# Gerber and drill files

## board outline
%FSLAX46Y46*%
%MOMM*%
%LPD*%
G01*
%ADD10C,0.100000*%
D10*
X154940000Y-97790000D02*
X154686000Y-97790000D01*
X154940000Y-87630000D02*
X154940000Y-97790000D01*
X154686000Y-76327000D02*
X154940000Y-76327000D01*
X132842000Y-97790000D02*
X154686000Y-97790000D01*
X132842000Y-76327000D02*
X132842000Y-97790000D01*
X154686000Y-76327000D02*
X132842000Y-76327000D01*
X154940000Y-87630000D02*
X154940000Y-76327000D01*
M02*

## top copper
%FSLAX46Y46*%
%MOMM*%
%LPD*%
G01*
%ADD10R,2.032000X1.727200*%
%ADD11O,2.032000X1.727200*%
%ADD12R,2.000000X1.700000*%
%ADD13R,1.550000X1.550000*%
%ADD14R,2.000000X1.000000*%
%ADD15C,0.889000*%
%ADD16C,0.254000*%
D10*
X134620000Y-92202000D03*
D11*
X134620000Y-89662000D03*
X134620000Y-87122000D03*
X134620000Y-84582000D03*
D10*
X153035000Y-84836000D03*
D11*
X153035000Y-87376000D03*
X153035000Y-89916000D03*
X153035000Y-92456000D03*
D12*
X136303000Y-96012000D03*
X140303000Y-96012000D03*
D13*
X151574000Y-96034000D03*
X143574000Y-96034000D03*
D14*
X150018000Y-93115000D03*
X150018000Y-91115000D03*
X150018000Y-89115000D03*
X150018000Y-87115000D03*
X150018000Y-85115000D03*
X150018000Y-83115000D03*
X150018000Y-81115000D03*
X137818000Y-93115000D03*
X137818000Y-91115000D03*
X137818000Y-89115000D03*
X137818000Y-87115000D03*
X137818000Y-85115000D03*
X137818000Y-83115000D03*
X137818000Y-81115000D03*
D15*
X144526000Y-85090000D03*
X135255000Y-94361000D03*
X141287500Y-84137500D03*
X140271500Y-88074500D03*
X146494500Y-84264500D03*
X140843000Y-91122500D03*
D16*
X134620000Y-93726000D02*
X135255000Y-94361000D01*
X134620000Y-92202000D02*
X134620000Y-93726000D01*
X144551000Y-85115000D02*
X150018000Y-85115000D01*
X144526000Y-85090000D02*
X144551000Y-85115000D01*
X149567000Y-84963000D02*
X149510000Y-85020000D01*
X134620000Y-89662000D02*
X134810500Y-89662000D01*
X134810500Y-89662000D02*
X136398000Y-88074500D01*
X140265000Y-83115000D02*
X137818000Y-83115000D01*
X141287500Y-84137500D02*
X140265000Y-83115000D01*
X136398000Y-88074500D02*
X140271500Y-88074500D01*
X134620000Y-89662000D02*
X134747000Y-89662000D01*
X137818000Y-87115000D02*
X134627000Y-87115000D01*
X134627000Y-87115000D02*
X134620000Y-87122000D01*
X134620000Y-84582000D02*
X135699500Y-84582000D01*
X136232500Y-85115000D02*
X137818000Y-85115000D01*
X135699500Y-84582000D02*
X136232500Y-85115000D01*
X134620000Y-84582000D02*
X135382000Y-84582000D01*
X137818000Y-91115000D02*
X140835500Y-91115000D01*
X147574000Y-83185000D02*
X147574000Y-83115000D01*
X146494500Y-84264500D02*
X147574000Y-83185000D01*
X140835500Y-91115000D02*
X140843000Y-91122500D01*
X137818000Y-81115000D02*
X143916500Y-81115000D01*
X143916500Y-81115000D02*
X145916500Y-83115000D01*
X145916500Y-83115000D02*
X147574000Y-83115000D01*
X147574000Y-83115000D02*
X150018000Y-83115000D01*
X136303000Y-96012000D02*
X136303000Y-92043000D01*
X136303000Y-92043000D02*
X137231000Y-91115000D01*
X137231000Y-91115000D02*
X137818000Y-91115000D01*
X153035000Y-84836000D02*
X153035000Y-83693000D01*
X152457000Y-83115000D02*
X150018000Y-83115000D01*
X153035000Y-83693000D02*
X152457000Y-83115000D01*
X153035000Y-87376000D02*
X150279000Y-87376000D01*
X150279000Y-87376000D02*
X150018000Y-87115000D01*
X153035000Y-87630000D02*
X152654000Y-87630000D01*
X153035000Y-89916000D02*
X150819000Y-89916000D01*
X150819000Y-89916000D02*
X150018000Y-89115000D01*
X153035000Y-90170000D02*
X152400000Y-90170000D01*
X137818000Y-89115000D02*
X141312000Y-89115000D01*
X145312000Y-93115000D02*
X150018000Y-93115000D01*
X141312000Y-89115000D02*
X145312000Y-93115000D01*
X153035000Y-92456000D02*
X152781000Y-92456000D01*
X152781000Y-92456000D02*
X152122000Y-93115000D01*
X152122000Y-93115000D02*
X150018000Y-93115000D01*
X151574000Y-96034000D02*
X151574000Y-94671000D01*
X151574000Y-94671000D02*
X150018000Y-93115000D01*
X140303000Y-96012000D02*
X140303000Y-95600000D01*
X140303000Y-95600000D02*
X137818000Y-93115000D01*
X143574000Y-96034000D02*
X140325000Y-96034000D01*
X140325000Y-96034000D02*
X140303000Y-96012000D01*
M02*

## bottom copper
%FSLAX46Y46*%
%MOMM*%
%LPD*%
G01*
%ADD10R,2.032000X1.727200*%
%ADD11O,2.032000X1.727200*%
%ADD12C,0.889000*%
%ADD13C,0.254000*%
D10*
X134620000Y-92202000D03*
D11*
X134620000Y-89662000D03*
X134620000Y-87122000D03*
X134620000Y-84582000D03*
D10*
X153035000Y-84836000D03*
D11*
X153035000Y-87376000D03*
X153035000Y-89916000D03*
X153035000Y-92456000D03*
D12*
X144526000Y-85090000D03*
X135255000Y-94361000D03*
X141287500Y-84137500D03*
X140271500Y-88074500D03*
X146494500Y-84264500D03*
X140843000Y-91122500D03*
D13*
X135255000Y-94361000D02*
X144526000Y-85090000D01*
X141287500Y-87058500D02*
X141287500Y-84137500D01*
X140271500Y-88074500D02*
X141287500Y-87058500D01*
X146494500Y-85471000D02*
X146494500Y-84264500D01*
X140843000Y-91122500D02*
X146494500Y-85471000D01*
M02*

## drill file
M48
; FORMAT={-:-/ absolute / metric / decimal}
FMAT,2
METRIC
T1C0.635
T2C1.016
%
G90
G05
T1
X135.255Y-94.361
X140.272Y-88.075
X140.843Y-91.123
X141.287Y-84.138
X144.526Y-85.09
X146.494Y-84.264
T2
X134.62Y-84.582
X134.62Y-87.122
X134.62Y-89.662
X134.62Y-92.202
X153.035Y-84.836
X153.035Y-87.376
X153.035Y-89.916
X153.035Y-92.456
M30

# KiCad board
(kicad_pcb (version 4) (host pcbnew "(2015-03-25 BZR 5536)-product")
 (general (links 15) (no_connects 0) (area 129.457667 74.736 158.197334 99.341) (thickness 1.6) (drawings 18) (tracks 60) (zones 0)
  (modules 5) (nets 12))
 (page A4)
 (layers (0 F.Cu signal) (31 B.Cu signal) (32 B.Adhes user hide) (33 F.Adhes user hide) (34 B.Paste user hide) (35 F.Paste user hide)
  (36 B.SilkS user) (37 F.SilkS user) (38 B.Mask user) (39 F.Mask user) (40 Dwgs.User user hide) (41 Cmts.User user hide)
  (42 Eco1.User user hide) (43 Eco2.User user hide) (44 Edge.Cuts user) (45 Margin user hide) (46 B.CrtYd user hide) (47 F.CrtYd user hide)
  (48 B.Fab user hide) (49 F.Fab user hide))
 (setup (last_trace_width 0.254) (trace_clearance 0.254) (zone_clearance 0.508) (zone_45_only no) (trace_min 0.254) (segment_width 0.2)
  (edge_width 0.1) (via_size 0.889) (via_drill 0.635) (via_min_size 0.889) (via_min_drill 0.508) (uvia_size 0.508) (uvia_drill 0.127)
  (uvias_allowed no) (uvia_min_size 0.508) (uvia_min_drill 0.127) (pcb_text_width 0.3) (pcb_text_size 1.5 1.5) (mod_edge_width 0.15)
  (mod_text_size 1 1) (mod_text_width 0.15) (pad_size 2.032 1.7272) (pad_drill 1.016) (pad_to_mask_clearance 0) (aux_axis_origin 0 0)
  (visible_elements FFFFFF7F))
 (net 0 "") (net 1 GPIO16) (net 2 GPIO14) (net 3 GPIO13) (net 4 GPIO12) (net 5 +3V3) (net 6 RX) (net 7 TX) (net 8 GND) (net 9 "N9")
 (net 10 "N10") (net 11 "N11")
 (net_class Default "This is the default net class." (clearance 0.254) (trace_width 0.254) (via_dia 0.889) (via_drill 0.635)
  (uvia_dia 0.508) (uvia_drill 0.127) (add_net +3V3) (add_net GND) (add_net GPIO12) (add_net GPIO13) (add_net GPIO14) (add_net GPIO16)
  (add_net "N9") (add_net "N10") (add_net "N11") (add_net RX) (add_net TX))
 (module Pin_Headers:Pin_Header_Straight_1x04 (layer F.Cu) (at 134.62 92.202 180)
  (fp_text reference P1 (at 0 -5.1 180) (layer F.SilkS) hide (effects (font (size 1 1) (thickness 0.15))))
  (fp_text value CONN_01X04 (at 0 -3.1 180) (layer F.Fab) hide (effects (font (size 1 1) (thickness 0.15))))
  (pad 1 thru_hole rect (at 0 0 180) (size 2.032 1.7272) (drill 1.016) (layers *.Cu *.Mask F.SilkS) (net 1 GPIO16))
  (pad 2 thru_hole oval (at 0 2.54 180) (size 2.032 1.7272) (drill 1.016) (layers *.Cu *.Mask F.SilkS) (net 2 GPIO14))
  (pad 3 thru_hole oval (at 0 5.08 180) (size 2.032 1.7272) (drill 1.016) (layers *.Cu *.Mask F.SilkS) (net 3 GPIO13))
  (pad 4 thru_hole oval (at 0 7.62 180) (size 2.032 1.7272) (drill 1.016) (layers *.Cu *.Mask F.SilkS) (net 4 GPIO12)))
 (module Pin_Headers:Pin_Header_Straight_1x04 (layer F.Cu) (at 153.035 84.836)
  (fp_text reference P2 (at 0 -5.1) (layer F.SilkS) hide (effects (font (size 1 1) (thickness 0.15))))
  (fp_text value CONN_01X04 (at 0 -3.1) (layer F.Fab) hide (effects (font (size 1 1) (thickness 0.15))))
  (pad 1 thru_hole rect (at 0 0) (size 2.032 1.7272) (drill 1.016) (layers *.Cu *.Mask F.SilkS) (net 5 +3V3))
  (pad 2 thru_hole oval (at 0 2.54) (size 2.032 1.7272) (drill 1.016) (layers *.Cu *.Mask F.SilkS) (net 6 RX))
  (pad 3 thru_hole oval (at 0 5.08) (size 2.032 1.7272) (drill 1.016) (layers *.Cu *.Mask F.SilkS) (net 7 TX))
  (pad 4 thru_hole oval (at 0 7.62) (size 2.032 1.7272) (drill 1.016) (layers *.Cu *.Mask F.SilkS) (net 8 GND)))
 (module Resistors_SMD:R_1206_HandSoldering (layer F.Cu) (at 138.303 96.012)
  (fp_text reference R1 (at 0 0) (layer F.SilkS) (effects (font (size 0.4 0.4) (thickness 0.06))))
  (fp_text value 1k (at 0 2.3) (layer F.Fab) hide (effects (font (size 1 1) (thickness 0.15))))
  (pad 1 smd rect (at -2 0) (size 2 1.7) (layers F.Cu F.Paste F.Mask) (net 5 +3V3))
  (pad 2 smd rect (at 2 0) (size 2 1.7) (layers F.Cu F.Paste F.Mask) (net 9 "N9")))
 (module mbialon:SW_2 (layer F.Cu) (at 147.574 94.234 180)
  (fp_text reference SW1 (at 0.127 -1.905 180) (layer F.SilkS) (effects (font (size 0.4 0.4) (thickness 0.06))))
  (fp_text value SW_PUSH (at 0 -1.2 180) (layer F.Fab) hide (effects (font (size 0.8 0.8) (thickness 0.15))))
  (pad 1 smd rect (at -4 -1.8 180) (size 1.55 1.55) (layers F.Cu F.Paste F.Mask) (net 8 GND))
  (pad 2 smd rect (at 4 -1.8 180) (size 1.55 1.55) (layers F.Cu F.Paste F.Mask) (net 9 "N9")))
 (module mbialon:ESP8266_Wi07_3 (layer F.Cu) (at 144.018 81.915)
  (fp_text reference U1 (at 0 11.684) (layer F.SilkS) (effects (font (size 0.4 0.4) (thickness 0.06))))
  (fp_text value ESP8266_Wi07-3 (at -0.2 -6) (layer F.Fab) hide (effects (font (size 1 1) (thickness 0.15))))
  (pad 1 smd rect (at 6 11.2) (size 2 1) (layers F.Cu F.Paste F.Mask) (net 8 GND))
  (pad 2 smd rect (at 6 9.2) (size 2 1) (layers F.Cu F.Paste F.Mask) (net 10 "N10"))
  (pad 3 smd rect (at 6 7.2) (size 2 1) (layers F.Cu F.Paste F.Mask) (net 7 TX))
  (pad 4 smd rect (at 6 5.2) (size 2 1) (layers F.Cu F.Paste F.Mask) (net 6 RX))
  (pad 5 smd rect (at 6 3.2) (size 2 1) (layers F.Cu F.Paste F.Mask) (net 1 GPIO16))
  (pad 6 smd rect (at 6 1.2) (size 2 1) (layers F.Cu F.Paste F.Mask) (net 5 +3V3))
  (pad 7 smd rect (at 6 -0.8) (size 2 1) (layers F.Cu F.Paste F.Mask) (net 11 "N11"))
  (pad 14 smd rect (at -6.2 11.2) (size 2 1) (layers F.Cu F.Paste F.Mask) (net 9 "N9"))
  (pad 13 smd rect (at -6.2 9.2) (size 2 1) (layers F.Cu F.Paste F.Mask) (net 5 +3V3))
  (pad 12 smd rect (at -6.2 7.2) (size 2 1) (layers F.Cu F.Paste F.Mask) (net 8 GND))
  (pad 11 smd rect (at -6.2 5.2) (size 2 1) (layers F.Cu F.Paste F.Mask) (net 3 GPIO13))
  (pad 10 smd rect (at -6.2 3.2) (size 2 1) (layers F.Cu F.Paste F.Mask) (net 4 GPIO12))
  (pad 9 smd rect (at -6.2 1.2) (size 2 1) (layers F.Cu F.Paste F.Mask) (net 2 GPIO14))
  (pad 8 smd rect (at -6.2 -0.8) (size 2 1) (layers F.Cu F.Paste F.Mask) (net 5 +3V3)))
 (gr_line (start 154.94 97.79) (end 154.686 97.79) (angle 90) (layer Edge.Cuts) (width 0.1))
 (gr_line (start 154.94 87.63) (end 154.94 97.79) (angle 90) (layer Edge.Cuts) (width 0.1))
 (gr_line (start 154.686 76.327) (end 154.94 76.327) (angle 90) (layer Edge.Cuts) (width 0.1))
 (gr_line (start 132.842 97.79) (end 154.686 97.79) (angle 90) (layer Edge.Cuts) (width 0.1))
 (gr_line (start 132.842 76.327) (end 132.842 97.79) (angle 90) (layer Edge.Cuts) (width 0.1))
 (gr_line (start 154.686 76.327) (end 132.842 76.327) (angle 90) (layer Edge.Cuts) (width 0.1))
 (gr_line (start 154.94 87.63) (end 154.94 76.327) (angle 90) (layer Edge.Cuts) (width 0.1))
 (via (at 144.526 85.09) (size 0.889) (layers F.Cu B.Cu) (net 1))
 (via (at 135.255 94.361) (size 0.889) (layers F.Cu B.Cu) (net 1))
 (via (at 141.2875 84.1375) (size 0.889) (layers F.Cu B.Cu) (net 2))
 (via (at 140.2715 88.0745) (size 0.889) (layers F.Cu B.Cu) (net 2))
 (via (at 146.4945 84.2645) (size 0.889) (layers F.Cu B.Cu) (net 5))
 (via (at 140.843 91.1225) (size 0.889) (layers F.Cu B.Cu) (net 5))
 (segment (start 134.62 93.726) (end 135.255 94.361) (width 0.254) (layer F.Cu) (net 1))
 (segment (start 135.255 94.361) (end 144.526 85.09) (width 0.254) (layer B.Cu) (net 1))
 (segment (start 134.62 92.202) (end 134.62 93.726) (width 0.254) (layer F.Cu) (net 1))
 (segment (start 144.551 85.115) (end 150.018 85.115) (width 0.254) (layer F.Cu) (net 1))
 (segment (start 144.526 85.09) (end 144.551 85.115) (width 0.254) (layer F.Cu) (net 1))
 (segment (start 149.567 84.963) (end 149.51 85.02) (width 0.254) (layer F.Cu) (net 1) (status 30))
 (segment (start 134.62 89.662) (end 134.8105 89.662) (width 0.254) (layer F.Cu) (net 2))
 (segment (start 134.8105 89.662) (end 136.398 88.0745) (width 0.254) (layer F.Cu) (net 2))
 (segment (start 140.265 83.115) (end 137.818 83.115) (width 0.254) (layer F.Cu) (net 2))
 (segment (start 141.2875 84.1375) (end 140.265 83.115) (width 0.254) (layer F.Cu) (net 2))
 (segment (start 141.2875 87.0585) (end 141.2875 84.1375) (width 0.254) (layer B.Cu) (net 2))
 (segment (start 140.2715 88.0745) (end 141.2875 87.0585) (width 0.254) (layer B.Cu) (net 2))
 (segment (start 136.398 88.0745) (end 140.2715 88.0745) (width 0.254) (layer F.Cu) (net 2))
 (segment (start 134.62 89.662) (end 134.747 89.662) (width 0.254) (layer F.Cu) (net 2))
 (segment (start 137.818 87.115) (end 134.627 87.115) (width 0.254) (layer F.Cu) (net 3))
 (segment (start 134.627 87.115) (end 134.62 87.122) (width 0.254) (layer F.Cu) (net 3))
 (segment (start 134.62 84.582) (end 135.6995 84.582) (width 0.254) (layer F.Cu) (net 4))
 (segment (start 136.2325 85.115) (end 137.818 85.115) (width 0.254) (layer F.Cu) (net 4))
 (segment (start 135.6995 84.582) (end 136.2325 85.115) (width 0.254) (layer F.Cu) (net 4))
 (segment (start 134.62 84.582) (end 135.382 84.582) (width 0.254) (layer F.Cu) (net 4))
 (segment (start 137.818 91.115) (end 140.8355 91.115) (width 0.254) (layer F.Cu) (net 5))
 (segment (start 147.574 83.185) (end 147.574 83.115) (width 0.254) (layer F.Cu) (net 5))
 (segment (start 146.4945 84.2645) (end 147.574 83.185) (width 0.254) (layer F.Cu) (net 5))
 (segment (start 146.4945 85.471) (end 146.4945 84.2645) (width 0.254) (layer B.Cu) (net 5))
 (segment (start 140.843 91.1225) (end 146.4945 85.471) (width 0.254) (layer B.Cu) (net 5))
 (segment (start 140.8355 91.115) (end 140.843 91.1225) (width 0.254) (layer F.Cu) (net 5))
 (segment (start 137.818 81.115) (end 143.9165 81.115) (width 0.254) (layer F.Cu) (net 5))
 (segment (start 143.9165 81.115) (end 145.9165 83.115) (width 0.254) (layer F.Cu) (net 5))
 (segment (start 145.9165 83.115) (end 147.574 83.115) (width 0.254) (layer F.Cu) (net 5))
 (segment (start 147.574 83.115) (end 150.018 83.115) (width 0.254) (layer F.Cu) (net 5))
 (segment (start 136.303 96.012) (end 136.303 92.043) (width 0.254) (layer F.Cu) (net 5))
 (segment (start 136.303 92.043) (end 137.231 91.115) (width 0.254) (layer F.Cu) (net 5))
 (segment (start 137.231 91.115) (end 137.818 91.115) (width 0.254) (layer F.Cu) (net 5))
 (segment (start 153.035 84.836) (end 153.035 83.693) (width 0.254) (layer F.Cu) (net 5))
 (segment (start 152.457 83.115) (end 150.018 83.115) (width 0.254) (layer F.Cu) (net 5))
 (segment (start 153.035 83.693) (end 152.457 83.115) (width 0.254) (layer F.Cu) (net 5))
 (segment (start 153.035 87.376) (end 150.279 87.376) (width 0.254) (layer F.Cu) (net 6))
 (segment (start 150.279 87.376) (end 150.018 87.115) (width 0.254) (layer F.Cu) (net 6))
 (segment (start 153.035 87.63) (end 152.654 87.63) (width 0.254) (layer F.Cu) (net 6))
 (segment (start 153.035 89.916) (end 150.819 89.916) (width 0.254) (layer F.Cu) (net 7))
 (segment (start 150.819 89.916) (end 150.018 89.115) (width 0.254) (layer F.Cu) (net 7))
 (segment (start 153.035 90.17) (end 152.4 90.17) (width 0.254) (layer F.Cu) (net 7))
 (segment (start 137.818 89.115) (end 141.312 89.115) (width 0.254) (layer F.Cu) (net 8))
 (segment (start 145.312 93.115) (end 150.018 93.115) (width 0.254) (layer F.Cu) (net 8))
 (segment (start 141.312 89.115) (end 145.312 93.115) (width 0.254) (layer F.Cu) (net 8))
 (segment (start 153.035 92.456) (end 152.781 92.456) (width 0.254) (layer F.Cu) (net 8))
 (segment (start 152.781 92.456) (end 152.122 93.115) (width 0.254) (layer F.Cu) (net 8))
 (segment (start 152.122 93.115) (end 150.018 93.115) (width 0.254) (layer F.Cu) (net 8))
 (segment (start 151.574 96.034) (end 151.574 94.671) (width 0.254) (layer F.Cu) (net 8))
 (segment (start 151.574 94.671) (end 150.018 93.115) (width 0.254) (layer F.Cu) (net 8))
 (segment (start 140.303 96.012) (end 140.303 95.6) (width 0.254) (layer F.Cu) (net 9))
 (segment (start 140.303 95.6) (end 137.818 93.115) (width 0.254) (layer F.Cu) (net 9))
 (segment (start 143.574 96.034) (end 140.325 96.034) (width 0.254) (layer F.Cu) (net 9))
 (segment (start 140.325 96.034) (end 140.303 96.012) (width 0.254) (layer F.Cu) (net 9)))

